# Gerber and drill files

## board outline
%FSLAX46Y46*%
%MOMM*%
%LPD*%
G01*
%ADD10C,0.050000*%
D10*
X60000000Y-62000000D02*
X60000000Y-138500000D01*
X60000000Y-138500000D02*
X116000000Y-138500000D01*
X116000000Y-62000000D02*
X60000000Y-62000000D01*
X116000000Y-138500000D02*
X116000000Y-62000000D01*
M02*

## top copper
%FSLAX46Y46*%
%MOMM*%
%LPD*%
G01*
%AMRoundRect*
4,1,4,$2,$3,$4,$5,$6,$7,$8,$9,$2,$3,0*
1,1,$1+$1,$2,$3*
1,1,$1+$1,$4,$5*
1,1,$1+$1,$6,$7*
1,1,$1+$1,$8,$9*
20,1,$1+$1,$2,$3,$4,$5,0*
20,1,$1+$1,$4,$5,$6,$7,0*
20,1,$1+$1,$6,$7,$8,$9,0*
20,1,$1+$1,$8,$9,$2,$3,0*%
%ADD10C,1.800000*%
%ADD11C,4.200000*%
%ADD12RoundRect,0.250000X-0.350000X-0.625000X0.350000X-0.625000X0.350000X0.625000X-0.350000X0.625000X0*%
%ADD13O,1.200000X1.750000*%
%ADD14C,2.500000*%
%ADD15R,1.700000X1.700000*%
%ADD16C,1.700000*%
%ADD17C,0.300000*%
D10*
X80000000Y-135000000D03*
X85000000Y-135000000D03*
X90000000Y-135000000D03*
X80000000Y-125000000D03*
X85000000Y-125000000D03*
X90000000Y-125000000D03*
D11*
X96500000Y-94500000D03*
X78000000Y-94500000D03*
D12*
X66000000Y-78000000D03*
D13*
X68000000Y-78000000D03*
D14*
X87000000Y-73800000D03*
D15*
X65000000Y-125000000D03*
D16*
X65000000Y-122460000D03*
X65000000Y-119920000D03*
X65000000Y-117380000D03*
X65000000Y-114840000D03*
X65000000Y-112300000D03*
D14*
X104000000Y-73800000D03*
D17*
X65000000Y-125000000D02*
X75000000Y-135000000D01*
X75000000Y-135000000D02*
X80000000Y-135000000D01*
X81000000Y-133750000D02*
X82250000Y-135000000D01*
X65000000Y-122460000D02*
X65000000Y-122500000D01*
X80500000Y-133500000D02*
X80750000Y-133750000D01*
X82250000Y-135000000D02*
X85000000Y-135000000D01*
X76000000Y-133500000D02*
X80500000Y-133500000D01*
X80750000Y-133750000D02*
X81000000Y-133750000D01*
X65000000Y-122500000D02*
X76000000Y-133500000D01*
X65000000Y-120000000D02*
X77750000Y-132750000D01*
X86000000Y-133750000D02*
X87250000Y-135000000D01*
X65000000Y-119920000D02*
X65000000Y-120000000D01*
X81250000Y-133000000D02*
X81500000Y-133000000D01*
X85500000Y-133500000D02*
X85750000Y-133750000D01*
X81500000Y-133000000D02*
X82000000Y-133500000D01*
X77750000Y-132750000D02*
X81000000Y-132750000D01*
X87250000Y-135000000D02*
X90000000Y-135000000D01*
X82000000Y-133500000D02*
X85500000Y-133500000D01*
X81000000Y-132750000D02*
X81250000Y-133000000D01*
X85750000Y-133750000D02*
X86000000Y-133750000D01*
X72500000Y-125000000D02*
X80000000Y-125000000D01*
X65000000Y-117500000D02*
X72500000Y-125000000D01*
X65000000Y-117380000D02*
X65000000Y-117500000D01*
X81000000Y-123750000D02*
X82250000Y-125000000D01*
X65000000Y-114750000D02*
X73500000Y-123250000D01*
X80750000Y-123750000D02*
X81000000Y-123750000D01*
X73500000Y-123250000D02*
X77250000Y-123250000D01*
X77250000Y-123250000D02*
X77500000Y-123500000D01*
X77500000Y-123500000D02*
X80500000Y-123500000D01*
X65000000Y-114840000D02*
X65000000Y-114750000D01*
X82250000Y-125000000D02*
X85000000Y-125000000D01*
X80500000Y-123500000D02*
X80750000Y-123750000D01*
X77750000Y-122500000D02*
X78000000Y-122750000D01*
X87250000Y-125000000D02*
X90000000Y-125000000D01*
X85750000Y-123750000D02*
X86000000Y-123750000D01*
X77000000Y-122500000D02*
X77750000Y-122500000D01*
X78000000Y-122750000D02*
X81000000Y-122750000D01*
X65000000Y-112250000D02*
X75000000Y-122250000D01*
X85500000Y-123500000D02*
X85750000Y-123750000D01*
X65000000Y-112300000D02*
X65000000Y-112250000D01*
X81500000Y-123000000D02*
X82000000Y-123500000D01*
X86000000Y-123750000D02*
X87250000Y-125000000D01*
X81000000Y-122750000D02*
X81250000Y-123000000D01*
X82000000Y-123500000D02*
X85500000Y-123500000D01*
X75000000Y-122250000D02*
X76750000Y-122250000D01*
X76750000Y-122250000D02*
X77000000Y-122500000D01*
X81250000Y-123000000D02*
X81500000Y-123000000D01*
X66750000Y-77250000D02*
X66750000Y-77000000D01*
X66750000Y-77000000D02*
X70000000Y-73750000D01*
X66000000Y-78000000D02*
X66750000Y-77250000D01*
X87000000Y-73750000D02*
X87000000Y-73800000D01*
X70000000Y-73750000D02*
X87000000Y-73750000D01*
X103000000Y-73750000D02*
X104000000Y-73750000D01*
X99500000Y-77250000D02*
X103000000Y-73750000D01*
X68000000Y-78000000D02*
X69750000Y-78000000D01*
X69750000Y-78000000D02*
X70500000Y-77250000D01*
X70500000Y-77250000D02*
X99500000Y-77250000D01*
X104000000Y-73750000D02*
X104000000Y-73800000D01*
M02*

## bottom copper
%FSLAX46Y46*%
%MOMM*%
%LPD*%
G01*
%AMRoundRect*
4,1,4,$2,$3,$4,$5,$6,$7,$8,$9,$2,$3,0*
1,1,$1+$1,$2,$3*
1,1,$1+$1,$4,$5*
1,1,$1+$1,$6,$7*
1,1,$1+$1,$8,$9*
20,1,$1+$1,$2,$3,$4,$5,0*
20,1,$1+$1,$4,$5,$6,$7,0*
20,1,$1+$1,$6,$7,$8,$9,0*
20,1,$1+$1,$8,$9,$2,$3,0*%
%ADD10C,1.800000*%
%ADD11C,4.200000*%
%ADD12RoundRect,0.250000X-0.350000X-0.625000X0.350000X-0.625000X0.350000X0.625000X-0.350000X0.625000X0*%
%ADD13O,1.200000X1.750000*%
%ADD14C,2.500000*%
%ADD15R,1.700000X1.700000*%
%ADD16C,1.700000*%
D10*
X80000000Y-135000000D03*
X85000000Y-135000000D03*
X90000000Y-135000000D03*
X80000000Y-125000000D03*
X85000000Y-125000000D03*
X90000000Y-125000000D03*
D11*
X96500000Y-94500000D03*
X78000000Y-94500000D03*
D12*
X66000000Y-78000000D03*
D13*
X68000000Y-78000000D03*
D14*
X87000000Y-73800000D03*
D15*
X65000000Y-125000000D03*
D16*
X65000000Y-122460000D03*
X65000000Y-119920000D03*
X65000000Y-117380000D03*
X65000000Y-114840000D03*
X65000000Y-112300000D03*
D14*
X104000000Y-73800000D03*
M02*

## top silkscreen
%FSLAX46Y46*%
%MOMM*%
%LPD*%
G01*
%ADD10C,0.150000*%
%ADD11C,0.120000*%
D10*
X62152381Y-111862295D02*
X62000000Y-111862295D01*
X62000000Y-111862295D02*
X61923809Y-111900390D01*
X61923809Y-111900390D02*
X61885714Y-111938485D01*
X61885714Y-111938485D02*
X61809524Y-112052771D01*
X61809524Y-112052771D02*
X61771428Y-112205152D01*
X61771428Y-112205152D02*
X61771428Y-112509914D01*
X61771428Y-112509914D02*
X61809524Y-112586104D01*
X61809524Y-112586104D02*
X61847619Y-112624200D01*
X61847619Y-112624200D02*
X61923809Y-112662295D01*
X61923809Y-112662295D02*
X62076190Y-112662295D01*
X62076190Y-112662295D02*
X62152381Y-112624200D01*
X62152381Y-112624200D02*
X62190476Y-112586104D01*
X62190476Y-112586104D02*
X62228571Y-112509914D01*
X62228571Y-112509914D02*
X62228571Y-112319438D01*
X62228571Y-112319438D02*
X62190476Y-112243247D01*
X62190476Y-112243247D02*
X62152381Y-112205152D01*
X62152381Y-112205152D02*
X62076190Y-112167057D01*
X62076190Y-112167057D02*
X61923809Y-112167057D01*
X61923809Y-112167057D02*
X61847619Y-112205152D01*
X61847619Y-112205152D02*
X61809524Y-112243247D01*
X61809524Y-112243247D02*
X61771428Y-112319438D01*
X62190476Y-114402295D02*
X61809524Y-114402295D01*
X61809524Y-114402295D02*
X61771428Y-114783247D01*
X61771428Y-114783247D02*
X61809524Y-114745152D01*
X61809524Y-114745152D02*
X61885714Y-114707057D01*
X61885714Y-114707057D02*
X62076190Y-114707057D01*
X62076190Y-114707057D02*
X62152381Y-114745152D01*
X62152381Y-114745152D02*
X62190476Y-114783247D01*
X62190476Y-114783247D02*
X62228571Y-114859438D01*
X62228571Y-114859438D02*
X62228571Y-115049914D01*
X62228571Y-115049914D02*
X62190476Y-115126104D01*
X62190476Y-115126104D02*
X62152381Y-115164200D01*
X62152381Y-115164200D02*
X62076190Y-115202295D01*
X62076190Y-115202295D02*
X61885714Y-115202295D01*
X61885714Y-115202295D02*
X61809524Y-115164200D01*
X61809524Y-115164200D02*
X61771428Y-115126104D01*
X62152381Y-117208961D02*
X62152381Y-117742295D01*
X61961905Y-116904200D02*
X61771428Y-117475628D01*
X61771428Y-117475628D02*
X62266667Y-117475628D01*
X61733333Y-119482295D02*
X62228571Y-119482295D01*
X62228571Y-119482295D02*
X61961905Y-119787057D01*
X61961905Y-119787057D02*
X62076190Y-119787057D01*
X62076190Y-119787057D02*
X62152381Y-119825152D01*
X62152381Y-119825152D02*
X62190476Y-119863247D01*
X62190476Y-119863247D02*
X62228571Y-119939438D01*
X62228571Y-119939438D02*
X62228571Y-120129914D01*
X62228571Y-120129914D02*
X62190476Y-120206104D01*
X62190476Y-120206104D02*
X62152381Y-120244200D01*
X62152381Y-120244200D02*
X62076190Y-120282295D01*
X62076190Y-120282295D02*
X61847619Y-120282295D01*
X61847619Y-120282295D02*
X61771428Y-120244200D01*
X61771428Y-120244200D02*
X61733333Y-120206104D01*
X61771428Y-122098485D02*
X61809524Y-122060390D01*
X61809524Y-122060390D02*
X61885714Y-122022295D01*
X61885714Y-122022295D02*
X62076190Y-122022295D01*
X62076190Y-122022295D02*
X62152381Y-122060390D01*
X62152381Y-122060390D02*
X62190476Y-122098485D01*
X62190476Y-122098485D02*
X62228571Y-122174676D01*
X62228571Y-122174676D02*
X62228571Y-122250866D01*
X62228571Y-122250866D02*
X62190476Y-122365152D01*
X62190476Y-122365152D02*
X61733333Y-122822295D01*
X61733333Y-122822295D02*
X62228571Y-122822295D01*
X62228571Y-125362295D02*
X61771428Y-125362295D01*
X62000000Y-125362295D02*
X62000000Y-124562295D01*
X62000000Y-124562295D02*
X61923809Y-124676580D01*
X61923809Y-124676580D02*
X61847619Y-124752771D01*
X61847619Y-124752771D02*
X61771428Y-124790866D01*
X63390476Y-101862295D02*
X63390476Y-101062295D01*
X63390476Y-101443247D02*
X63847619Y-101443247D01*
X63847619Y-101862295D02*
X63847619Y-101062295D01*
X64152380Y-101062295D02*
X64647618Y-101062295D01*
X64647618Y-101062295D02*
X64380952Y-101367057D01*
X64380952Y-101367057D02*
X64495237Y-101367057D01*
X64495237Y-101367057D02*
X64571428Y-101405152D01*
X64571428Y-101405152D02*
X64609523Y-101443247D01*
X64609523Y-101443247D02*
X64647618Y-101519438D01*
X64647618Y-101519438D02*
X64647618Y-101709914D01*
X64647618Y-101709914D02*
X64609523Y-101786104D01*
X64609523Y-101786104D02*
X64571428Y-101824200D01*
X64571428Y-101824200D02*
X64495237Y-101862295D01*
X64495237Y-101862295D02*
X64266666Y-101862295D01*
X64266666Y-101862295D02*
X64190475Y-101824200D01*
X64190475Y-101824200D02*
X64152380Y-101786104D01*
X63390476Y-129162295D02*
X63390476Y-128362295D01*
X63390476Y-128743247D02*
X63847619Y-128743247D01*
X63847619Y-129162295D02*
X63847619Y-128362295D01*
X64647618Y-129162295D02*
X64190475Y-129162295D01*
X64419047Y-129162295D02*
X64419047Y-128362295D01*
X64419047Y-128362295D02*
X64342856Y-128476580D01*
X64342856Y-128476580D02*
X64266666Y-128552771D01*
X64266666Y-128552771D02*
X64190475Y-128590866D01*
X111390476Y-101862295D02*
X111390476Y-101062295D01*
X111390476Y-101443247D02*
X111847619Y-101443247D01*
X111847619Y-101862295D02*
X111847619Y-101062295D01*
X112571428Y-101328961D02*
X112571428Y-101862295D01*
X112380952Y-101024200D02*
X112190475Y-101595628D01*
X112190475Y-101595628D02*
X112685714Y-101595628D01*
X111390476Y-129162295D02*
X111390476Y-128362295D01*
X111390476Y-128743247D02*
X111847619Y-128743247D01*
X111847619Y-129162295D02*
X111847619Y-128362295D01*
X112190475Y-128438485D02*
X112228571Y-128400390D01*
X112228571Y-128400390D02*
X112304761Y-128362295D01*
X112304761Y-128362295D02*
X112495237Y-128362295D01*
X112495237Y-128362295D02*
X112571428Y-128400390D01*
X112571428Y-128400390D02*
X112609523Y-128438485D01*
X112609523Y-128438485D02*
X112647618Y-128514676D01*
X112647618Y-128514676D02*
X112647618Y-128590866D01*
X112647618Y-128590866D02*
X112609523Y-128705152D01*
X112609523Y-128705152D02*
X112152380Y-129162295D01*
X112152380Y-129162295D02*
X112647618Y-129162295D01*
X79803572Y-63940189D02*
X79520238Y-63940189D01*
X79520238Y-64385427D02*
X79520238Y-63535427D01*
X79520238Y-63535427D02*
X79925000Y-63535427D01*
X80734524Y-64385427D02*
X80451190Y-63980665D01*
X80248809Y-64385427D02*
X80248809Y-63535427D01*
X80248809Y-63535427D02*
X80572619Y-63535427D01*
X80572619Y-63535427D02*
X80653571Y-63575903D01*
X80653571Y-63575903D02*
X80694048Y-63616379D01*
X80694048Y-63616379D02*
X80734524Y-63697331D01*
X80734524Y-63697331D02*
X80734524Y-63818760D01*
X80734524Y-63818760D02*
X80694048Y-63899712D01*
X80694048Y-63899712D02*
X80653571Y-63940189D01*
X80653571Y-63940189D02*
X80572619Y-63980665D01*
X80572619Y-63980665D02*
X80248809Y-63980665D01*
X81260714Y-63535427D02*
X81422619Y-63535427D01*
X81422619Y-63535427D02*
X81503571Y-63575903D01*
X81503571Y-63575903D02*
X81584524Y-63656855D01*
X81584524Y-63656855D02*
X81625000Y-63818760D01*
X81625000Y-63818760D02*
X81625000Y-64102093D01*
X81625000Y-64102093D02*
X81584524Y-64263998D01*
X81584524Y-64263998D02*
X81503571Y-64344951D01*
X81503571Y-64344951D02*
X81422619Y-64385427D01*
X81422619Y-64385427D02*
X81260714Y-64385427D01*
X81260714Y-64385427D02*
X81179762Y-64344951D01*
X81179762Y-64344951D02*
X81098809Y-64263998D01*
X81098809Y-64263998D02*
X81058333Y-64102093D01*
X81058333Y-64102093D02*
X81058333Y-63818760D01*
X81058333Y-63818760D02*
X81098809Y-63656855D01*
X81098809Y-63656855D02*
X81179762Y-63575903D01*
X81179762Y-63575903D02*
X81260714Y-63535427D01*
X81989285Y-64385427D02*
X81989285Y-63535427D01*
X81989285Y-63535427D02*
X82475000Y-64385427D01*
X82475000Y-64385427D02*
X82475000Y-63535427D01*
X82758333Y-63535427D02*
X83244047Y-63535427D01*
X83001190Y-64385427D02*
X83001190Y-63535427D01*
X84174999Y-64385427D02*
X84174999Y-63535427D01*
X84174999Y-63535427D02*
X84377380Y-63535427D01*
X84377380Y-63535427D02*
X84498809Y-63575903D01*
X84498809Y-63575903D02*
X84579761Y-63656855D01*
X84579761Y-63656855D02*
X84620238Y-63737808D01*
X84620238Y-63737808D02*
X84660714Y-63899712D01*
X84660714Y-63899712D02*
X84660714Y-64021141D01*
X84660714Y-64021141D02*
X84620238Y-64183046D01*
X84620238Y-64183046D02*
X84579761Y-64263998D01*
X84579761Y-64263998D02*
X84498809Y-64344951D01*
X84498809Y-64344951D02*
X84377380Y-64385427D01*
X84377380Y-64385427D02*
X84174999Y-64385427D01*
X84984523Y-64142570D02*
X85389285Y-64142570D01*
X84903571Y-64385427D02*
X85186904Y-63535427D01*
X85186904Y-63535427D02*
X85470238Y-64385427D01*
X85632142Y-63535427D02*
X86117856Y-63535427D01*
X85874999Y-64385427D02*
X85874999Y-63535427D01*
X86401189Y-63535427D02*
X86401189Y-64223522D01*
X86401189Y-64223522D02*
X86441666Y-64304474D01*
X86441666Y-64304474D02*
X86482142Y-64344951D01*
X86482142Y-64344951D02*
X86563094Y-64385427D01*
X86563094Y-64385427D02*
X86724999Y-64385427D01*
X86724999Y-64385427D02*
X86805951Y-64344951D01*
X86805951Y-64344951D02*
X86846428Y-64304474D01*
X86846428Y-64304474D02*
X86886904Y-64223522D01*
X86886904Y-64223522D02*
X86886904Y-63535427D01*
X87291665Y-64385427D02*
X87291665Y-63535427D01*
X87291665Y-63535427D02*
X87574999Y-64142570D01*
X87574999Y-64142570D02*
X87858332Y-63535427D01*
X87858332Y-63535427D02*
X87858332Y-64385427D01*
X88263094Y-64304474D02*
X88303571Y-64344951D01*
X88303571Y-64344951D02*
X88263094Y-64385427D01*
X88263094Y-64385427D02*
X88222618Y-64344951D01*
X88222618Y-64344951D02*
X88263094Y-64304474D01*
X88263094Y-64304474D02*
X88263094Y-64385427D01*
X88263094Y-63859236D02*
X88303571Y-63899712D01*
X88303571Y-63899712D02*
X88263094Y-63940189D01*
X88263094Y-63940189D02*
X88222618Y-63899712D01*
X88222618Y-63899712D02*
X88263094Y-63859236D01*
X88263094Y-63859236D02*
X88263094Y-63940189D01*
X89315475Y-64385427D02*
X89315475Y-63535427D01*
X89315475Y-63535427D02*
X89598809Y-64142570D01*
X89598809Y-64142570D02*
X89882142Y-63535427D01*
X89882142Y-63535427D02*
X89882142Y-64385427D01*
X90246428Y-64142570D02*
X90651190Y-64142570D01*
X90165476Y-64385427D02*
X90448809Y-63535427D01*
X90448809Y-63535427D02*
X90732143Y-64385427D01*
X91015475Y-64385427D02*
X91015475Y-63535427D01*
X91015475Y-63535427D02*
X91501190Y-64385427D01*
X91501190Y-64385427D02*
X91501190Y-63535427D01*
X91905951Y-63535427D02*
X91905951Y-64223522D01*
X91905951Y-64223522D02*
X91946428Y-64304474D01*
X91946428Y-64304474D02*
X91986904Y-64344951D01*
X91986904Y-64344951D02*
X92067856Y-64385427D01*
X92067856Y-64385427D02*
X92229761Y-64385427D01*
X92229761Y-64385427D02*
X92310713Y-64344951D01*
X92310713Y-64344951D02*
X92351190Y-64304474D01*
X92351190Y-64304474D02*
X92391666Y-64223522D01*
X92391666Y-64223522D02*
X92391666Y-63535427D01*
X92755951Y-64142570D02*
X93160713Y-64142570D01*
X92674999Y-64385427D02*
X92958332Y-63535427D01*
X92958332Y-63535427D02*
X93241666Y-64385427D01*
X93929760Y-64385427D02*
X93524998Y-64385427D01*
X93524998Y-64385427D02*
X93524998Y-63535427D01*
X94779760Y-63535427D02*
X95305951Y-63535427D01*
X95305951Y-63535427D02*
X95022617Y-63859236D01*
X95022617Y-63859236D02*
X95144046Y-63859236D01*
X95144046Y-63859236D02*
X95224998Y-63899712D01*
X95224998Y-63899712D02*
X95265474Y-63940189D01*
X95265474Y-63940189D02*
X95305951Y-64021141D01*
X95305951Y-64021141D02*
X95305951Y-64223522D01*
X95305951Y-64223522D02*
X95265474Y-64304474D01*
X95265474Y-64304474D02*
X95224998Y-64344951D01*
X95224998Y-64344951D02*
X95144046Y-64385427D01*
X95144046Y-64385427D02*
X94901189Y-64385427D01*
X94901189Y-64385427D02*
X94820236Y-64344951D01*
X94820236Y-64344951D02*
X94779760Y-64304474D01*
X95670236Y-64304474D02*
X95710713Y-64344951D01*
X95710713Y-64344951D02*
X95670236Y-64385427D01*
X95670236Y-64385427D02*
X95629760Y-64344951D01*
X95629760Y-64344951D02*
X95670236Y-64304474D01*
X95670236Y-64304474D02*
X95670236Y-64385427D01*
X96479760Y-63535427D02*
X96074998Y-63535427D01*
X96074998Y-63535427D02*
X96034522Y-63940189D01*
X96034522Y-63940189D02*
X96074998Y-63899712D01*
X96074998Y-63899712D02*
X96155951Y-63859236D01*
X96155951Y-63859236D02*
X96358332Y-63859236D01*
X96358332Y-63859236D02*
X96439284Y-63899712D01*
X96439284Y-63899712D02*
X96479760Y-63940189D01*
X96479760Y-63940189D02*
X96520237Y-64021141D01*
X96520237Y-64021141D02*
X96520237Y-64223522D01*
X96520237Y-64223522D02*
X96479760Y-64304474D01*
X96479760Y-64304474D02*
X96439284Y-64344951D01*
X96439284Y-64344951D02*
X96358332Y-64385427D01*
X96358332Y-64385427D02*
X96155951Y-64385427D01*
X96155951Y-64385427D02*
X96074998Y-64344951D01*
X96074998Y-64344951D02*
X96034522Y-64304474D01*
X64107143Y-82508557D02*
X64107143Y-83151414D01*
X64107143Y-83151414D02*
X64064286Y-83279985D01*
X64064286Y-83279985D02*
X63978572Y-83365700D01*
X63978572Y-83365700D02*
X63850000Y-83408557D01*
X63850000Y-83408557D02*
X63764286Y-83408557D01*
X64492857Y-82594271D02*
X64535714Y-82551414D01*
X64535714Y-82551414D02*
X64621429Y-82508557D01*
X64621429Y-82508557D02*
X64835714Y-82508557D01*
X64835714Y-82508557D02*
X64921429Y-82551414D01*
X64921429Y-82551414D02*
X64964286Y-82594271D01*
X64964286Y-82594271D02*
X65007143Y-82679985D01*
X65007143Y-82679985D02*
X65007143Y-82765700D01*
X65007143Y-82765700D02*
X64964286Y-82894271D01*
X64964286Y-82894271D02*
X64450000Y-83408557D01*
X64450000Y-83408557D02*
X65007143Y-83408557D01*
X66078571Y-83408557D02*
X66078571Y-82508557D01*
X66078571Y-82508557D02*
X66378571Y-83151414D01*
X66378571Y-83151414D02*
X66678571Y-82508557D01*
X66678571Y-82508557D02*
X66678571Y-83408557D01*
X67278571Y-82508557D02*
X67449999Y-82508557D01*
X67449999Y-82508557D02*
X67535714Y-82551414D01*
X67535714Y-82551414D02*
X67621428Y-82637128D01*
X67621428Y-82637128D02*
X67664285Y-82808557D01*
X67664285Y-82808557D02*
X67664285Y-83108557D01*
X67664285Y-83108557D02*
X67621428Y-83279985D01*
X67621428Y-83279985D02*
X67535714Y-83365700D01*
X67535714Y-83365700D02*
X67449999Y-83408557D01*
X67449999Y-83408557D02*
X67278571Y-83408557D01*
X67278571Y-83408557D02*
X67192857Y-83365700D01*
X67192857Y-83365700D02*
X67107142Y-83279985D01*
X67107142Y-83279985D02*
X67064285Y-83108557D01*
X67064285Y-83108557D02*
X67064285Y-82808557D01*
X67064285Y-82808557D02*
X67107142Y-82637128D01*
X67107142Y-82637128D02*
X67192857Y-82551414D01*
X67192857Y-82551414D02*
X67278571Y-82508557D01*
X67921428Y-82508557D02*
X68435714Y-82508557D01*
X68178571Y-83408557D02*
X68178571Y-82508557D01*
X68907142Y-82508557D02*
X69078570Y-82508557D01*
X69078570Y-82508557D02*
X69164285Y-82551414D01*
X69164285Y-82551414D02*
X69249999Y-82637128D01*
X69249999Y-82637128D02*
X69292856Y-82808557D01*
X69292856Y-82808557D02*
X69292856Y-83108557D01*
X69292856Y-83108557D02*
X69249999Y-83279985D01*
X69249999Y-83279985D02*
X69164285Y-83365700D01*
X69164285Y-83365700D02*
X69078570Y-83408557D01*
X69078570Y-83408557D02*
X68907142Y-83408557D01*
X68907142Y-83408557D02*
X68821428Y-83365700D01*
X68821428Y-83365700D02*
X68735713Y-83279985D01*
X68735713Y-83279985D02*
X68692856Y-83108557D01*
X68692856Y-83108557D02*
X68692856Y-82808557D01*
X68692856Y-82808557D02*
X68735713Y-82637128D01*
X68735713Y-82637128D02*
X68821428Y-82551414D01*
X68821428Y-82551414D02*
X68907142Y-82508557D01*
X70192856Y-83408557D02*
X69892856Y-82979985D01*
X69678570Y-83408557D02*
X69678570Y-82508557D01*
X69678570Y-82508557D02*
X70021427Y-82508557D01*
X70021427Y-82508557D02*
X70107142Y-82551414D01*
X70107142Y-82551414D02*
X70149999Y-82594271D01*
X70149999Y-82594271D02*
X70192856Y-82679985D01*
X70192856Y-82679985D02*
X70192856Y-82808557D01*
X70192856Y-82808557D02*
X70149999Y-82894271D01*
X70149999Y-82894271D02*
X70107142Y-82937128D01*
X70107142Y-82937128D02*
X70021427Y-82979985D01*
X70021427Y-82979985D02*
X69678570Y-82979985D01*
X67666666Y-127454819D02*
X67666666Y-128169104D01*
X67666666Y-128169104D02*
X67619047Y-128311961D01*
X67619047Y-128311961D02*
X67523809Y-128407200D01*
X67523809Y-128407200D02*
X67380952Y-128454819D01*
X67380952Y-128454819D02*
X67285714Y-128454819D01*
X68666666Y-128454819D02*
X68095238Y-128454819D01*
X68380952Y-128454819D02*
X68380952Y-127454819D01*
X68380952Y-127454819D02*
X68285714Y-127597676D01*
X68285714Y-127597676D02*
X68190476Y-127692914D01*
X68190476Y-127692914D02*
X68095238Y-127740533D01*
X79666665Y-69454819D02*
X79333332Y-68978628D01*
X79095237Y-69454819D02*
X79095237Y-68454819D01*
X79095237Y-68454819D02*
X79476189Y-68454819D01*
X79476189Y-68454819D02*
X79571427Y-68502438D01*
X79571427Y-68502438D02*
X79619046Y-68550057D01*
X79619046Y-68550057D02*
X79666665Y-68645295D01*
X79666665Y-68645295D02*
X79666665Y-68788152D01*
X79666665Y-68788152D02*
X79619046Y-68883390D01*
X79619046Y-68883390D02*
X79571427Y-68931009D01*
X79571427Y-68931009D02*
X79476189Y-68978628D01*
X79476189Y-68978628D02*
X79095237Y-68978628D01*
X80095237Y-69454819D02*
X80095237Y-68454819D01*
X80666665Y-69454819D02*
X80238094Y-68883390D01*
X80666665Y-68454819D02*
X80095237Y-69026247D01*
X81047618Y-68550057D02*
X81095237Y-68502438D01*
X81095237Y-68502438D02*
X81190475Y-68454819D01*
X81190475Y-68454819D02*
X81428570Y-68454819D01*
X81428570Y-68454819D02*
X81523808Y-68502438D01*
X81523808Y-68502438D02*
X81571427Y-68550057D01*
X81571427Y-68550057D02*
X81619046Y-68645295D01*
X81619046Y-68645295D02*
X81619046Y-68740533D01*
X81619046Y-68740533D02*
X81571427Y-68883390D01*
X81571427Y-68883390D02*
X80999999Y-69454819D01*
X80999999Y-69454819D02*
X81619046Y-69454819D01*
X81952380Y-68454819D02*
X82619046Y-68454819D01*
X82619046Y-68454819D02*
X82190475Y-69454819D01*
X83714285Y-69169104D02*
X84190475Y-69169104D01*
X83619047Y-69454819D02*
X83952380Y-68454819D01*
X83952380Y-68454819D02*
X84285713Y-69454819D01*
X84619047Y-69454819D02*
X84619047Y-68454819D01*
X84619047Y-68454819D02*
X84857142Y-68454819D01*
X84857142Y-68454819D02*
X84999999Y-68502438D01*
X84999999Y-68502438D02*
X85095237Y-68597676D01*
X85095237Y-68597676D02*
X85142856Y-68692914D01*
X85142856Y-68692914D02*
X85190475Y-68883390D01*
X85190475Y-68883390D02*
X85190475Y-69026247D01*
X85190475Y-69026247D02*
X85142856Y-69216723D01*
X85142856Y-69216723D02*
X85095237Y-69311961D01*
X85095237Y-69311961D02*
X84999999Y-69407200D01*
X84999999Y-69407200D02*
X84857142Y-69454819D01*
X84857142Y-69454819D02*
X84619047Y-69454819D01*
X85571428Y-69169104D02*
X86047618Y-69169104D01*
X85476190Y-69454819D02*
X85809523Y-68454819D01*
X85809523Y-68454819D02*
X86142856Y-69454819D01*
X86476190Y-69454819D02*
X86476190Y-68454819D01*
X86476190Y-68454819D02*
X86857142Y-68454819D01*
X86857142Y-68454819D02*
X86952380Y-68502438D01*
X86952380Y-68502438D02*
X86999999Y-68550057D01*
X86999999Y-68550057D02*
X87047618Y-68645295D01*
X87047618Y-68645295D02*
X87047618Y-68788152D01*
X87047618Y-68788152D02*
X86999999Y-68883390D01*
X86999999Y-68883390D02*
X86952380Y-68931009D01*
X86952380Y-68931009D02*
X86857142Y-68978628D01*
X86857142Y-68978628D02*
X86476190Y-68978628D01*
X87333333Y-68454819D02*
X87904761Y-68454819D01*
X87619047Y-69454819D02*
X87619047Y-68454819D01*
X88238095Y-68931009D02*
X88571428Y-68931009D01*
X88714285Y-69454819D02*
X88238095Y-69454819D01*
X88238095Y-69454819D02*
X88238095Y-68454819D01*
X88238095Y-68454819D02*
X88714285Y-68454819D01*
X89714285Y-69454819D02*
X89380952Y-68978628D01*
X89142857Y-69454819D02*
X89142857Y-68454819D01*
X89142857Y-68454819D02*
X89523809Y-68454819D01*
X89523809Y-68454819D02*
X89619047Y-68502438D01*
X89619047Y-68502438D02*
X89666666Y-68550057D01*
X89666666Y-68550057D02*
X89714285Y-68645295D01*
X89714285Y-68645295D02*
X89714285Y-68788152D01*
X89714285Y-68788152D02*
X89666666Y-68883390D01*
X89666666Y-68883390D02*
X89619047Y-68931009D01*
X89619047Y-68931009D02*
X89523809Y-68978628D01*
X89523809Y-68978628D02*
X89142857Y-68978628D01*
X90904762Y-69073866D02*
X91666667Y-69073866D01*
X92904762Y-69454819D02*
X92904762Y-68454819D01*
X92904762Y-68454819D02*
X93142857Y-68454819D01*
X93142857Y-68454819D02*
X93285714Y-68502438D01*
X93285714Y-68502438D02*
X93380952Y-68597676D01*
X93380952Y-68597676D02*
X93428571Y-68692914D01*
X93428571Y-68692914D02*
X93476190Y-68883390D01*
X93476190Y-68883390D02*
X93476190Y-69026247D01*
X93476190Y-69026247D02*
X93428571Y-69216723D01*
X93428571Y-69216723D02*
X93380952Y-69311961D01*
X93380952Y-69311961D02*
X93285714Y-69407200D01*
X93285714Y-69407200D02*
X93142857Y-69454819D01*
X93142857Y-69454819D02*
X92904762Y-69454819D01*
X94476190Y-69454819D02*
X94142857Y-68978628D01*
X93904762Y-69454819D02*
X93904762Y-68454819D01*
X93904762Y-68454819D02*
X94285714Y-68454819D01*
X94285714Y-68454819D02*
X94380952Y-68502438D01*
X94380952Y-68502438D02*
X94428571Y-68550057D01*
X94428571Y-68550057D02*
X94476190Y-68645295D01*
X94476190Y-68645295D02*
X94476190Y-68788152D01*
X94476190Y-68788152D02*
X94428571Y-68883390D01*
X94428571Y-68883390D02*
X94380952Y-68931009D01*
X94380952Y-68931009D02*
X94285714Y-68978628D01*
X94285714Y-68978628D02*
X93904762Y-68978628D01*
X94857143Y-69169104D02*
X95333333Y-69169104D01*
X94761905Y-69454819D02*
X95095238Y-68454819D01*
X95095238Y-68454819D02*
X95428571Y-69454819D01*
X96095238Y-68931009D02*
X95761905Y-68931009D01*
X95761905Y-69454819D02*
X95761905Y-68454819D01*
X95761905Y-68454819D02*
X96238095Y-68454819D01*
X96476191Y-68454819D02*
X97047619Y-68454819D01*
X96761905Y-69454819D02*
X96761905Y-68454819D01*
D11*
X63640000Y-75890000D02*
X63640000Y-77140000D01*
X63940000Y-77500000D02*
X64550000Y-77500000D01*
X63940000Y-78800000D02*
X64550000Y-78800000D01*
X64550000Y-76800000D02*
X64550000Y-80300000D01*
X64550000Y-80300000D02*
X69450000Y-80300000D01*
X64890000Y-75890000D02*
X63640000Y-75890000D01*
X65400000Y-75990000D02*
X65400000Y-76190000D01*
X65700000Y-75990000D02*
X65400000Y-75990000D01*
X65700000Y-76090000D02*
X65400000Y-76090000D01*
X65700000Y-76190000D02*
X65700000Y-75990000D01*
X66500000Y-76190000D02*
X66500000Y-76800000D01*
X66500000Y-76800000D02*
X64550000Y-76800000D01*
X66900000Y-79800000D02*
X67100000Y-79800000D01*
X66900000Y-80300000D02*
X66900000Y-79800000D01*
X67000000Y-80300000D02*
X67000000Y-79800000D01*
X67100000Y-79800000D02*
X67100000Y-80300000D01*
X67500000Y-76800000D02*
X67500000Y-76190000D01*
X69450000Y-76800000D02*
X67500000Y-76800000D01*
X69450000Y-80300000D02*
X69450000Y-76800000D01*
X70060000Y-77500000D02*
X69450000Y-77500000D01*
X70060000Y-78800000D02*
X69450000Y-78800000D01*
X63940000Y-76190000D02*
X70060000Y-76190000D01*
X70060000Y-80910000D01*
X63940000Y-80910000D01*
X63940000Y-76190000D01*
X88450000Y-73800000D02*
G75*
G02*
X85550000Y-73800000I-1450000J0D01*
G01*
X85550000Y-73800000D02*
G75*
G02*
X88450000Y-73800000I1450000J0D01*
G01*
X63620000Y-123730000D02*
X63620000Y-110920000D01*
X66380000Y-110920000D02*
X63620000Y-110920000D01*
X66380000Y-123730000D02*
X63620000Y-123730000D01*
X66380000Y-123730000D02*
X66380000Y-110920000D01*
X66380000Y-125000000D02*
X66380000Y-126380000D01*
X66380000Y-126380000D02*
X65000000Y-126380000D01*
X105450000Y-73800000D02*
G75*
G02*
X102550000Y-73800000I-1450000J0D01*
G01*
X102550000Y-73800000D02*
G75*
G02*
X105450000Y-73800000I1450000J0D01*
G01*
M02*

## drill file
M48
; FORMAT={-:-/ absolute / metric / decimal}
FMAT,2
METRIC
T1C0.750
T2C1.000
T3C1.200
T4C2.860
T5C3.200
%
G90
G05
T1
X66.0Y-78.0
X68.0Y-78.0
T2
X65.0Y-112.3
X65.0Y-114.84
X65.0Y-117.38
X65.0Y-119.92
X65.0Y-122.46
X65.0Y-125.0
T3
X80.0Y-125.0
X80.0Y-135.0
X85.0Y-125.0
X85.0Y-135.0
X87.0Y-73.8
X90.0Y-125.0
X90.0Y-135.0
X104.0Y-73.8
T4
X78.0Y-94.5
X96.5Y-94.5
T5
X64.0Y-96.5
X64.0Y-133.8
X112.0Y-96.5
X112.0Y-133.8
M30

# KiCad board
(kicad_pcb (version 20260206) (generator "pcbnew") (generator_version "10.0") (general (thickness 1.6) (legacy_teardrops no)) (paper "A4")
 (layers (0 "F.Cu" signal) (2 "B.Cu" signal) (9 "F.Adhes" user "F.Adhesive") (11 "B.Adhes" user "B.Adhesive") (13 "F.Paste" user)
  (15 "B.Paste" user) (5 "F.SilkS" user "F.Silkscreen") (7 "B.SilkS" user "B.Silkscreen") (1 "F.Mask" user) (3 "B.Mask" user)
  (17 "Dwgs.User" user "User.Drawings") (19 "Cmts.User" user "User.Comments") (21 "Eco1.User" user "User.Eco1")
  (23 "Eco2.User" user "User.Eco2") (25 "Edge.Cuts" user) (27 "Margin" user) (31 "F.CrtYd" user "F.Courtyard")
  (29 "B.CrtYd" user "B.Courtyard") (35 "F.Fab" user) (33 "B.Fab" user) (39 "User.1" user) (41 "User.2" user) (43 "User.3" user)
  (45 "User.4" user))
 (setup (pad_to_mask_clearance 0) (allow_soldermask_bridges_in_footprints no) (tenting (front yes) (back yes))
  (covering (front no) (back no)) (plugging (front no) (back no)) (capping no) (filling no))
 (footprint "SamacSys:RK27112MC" (layer "F.Cu") (at 85 94.5 -90)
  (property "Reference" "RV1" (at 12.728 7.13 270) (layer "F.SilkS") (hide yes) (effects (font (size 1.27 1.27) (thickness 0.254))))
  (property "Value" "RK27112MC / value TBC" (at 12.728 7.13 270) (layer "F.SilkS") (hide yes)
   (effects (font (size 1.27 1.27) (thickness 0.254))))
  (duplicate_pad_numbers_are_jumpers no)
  (pad "1" thru_hole circle (at 40.5 5 270) (size 1.8 1.8) (drill 1.2) (layers "*.Cu" "*.Mask") (remove_unused_layers no) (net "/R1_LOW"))
  (pad "2" thru_hole circle (at 40.5 0 270) (size 1.8 1.8) (drill 1.2) (layers "*.Cu" "*.Mask") (remove_unused_layers no) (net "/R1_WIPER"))
  (pad "3" thru_hole circle (at 40.5 -5 270) (size 1.8 1.8) (drill 1.2) (layers "*.Cu" "*.Mask") (remove_unused_layers no) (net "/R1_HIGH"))
  (pad "4" thru_hole circle (at 30.5 5 270) (size 1.8 1.8) (drill 1.2) (layers "*.Cu" "*.Mask") (remove_unused_layers no) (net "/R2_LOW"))
  (pad "5" thru_hole circle (at 30.5 0 270) (size 1.8 1.8) (drill 1.2) (layers "*.Cu" "*.Mask") (remove_unused_layers no) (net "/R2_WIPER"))
  (pad "6" thru_hole circle (at 30.5 -5 270) (size 1.8 1.8) (drill 1.2) (layers "*.Cu" "*.Mask") (remove_unused_layers no) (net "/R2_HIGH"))
  (pad "7" thru_hole circle (at 0 -11.5 270) (size 4.2 4.2) (drill 2.86) (layers "*.Cu" "*.Mask") (remove_unused_layers no)
   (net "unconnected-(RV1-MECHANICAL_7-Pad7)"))
  (pad "8" thru_hole circle (at 0 7 270) (size 4.2 4.2) (drill 2.86) (layers "*.Cu" "*.Mask") (remove_unused_layers no)
   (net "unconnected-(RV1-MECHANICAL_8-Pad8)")))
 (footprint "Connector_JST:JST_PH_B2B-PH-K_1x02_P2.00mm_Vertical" (layer "F.Cu") (at 66 78)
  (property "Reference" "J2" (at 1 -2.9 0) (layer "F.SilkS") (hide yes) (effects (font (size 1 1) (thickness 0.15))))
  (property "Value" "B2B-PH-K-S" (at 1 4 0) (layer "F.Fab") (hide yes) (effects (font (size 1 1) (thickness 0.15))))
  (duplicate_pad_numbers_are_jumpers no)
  (fp_line (start -2.36 -2.11) (end -2.36 -0.86) (stroke (width 0.12) (type solid)) (layer "F.SilkS"))
  (fp_line (start -2.06 -0.5) (end -1.45 -0.5) (stroke (width 0.12) (type solid)) (layer "F.SilkS"))
  (fp_line (start -2.06 0.8) (end -1.45 0.8) (stroke (width 0.12) (type solid)) (layer "F.SilkS"))
  (fp_line (start -1.45 -1.2) (end -1.45 2.3) (stroke (width 0.12) (type solid)) (layer "F.SilkS"))
  (fp_line (start -1.45 2.3) (end 3.45 2.3) (stroke (width 0.12) (type solid)) (layer "F.SilkS"))
  (fp_line (start -1.11 -2.11) (end -2.36 -2.11) (stroke (width 0.12) (type solid)) (layer "F.SilkS"))
  (fp_line (start -0.6 -2.01) (end -0.6 -1.81) (stroke (width 0.12) (type solid)) (layer "F.SilkS"))
  (fp_line (start -0.3 -2.01) (end -0.6 -2.01) (stroke (width 0.12) (type solid)) (layer "F.SilkS"))
  (fp_line (start -0.3 -1.91) (end -0.6 -1.91) (stroke (width 0.12) (type solid)) (layer "F.SilkS"))
  (fp_line (start -0.3 -1.81) (end -0.3 -2.01) (stroke (width 0.12) (type solid)) (layer "F.SilkS"))
  (fp_line (start 0.5 -1.81) (end 0.5 -1.2) (stroke (width 0.12) (type solid)) (layer "F.SilkS"))
  (fp_line (start 0.5 -1.2) (end -1.45 -1.2) (stroke (width 0.12) (type solid)) (layer "F.SilkS"))
  (fp_line (start 0.9 1.8) (end 1.1 1.8) (stroke (width 0.12) (type solid)) (layer "F.SilkS"))
  (fp_line (start 0.9 2.3) (end 0.9 1.8) (stroke (width 0.12) (type solid)) (layer "F.SilkS"))
  (fp_line (start 1 2.3) (end 1 1.8) (stroke (width 0.12) (type solid)) (layer "F.SilkS"))
  (fp_line (start 1.1 1.8) (end 1.1 2.3) (stroke (width 0.12) (type solid)) (layer "F.SilkS"))
  (fp_line (start 1.5 -1.2) (end 1.5 -1.81) (stroke (width 0.12) (type solid)) (layer "F.SilkS"))
  (fp_line (start 3.45 -1.2) (end 1.5 -1.2) (stroke (width 0.12) (type solid)) (layer "F.SilkS"))
  (fp_line (start 3.45 2.3) (end 3.45 -1.2) (stroke (width 0.12) (type solid)) (layer "F.SilkS"))
  (fp_line (start 4.06 -0.5) (end 3.45 -0.5) (stroke (width 0.12) (type solid)) (layer "F.SilkS"))
  (fp_line (start 4.06 0.8) (end 3.45 0.8) (stroke (width 0.12) (type solid)) (layer "F.SilkS"))
  (fp_rect (start -2.06 -1.81) (end 4.06 2.91) (stroke (width 0.12) (type solid)) (fill no) (layer "F.SilkS"))
  (pad "1" thru_hole roundrect (at 0 0) (size 1.2 1.75) (drill 0.75) (layers "*.Cu" "*.Mask") (remove_unused_layers no)
   (roundrect_rratio 0.208333) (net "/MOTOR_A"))
  (pad "2" thru_hole oval (at 2 0) (size 1.2 1.75) (drill 0.75) (layers "*.Cu" "*.Mask") (remove_unused_layers no) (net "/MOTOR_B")))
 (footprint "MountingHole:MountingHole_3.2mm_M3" (layer "F.Cu") (at 112 133.8)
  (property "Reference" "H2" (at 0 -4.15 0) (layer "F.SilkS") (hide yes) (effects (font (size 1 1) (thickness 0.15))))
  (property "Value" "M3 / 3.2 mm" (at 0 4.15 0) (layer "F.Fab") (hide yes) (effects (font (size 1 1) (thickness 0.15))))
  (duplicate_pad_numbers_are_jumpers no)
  (pad "" np_thru_hole circle (at 0 0) (size 3.2 3.2) (drill 3.2) (layers "*.Cu" "*.Mask")))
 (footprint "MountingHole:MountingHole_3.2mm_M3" (layer "F.Cu") (at 64 96.5)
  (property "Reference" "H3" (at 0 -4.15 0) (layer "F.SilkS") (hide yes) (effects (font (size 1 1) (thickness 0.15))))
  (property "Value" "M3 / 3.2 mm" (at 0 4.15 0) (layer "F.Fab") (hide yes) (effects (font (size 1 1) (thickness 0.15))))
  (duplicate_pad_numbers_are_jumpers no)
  (pad "" np_thru_hole circle (at 0 0) (size 3.2 3.2) (drill 3.2) (layers "*.Cu" "*.Mask")))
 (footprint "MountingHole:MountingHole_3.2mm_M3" (layer "F.Cu") (at 64 133.8)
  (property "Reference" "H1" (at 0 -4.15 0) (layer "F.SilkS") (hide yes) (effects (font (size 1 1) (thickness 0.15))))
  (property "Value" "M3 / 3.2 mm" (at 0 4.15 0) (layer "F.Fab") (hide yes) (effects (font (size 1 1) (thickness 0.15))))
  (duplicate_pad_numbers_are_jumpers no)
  (pad "" np_thru_hole circle (at 0 0) (size 3.2 3.2) (drill 3.2) (layers "*.Cu" "*.Mask")))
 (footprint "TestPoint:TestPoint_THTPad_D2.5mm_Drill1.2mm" (layer "F.Cu") (at 87 73.8)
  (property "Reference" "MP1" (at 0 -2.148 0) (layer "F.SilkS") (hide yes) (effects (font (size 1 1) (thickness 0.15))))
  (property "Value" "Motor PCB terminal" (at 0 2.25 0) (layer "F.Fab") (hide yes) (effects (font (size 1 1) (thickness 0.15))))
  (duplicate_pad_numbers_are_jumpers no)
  (fp_circle (center 0 0) (end 0 1.45) (stroke (width 0.12) (type solid)) (fill no) (layer "F.SilkS"))
  (pad "1" thru_hole circle (at 0 0) (size 2.5 2.5) (drill 1.2) (layers "*.Cu" "*.Mask") (remove_unused_layers no) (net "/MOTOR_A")))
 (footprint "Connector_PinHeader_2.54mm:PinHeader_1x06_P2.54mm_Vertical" (layer "F.Cu") (at 65 125 180)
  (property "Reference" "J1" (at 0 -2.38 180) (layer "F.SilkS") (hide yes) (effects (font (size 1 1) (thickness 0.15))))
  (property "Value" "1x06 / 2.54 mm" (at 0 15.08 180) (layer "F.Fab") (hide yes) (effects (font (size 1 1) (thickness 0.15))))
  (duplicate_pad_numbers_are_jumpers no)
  (fp_line (start 1.38 1.27) (end 1.38 14.08) (stroke (width 0.12) (type solid)) (layer "F.SilkS"))
  (fp_line (start -1.38 14.08) (end 1.38 14.08) (stroke (width 0.12) (type solid)) (layer "F.SilkS"))
  (fp_line (start -1.38 1.27) (end 1.38 1.27) (stroke (width 0.12) (type solid)) (layer "F.SilkS"))
  (fp_line (start -1.38 1.27) (end -1.38 14.08) (stroke (width 0.12) (type solid)) (layer "F.SilkS"))
  (fp_line (start -1.38 0) (end -1.38 -1.38) (stroke (width 0.12) (type solid)) (layer "F.SilkS"))
  (fp_line (start -1.38 -1.38) (end 0 -1.38) (stroke (width 0.12) (type solid)) (layer "F.SilkS"))
  (pad "1" thru_hole rect (at 0 0 180) (size 1.7 1.7) (drill 1) (layers "*.Cu" "*.Mask") (remove_unused_layers no) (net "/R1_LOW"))
  (pad "2" thru_hole circle (at 0 2.54 180) (size 1.7 1.7) (drill 1) (layers "*.Cu" "*.Mask") (remove_unused_layers no) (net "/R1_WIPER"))
  (pad "3" thru_hole circle (at 0 5.08 180) (size 1.7 1.7) (drill 1) (layers "*.Cu" "*.Mask") (remove_unused_layers no) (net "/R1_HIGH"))
  (pad "4" thru_hole circle (at 0 7.62 180) (size 1.7 1.7) (drill 1) (layers "*.Cu" "*.Mask") (remove_unused_layers no) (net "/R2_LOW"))
  (pad "5" thru_hole circle (at 0 10.16 180) (size 1.7 1.7) (drill 1) (layers "*.Cu" "*.Mask") (remove_unused_layers no) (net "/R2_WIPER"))
  (pad "6" thru_hole circle (at 0 12.7 180) (size 1.7 1.7) (drill 1) (layers "*.Cu" "*.Mask") (remove_unused_layers no) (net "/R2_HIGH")))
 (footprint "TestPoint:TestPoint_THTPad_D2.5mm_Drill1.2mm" (layer "F.Cu") (at 104 73.8)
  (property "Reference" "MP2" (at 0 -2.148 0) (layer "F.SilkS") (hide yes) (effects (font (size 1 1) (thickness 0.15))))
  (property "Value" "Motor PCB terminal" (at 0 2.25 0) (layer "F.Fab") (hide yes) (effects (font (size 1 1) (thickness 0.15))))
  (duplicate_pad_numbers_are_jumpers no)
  (fp_circle (center 0 0) (end 0 1.45) (stroke (width 0.12) (type solid)) (fill no) (layer "F.SilkS"))
  (pad "1" thru_hole circle (at 0 0) (size 2.5 2.5) (drill 1.2) (layers "*.Cu" "*.Mask") (remove_unused_layers no) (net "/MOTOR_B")))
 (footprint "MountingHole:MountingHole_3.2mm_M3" (layer "F.Cu") (at 112 96.5)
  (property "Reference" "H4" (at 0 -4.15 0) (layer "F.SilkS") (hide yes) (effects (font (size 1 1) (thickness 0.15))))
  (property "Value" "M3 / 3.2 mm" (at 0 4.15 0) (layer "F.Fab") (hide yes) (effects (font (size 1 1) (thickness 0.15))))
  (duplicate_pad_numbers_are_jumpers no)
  (pad "" np_thru_hole circle (at 0 0) (size 3.2 3.2) (drill 3.2) (layers "*.Cu" "*.Mask")))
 (gr_line (start 60 62) (end 60 138.5) (stroke (width 0.05) (type default)) (layer "Edge.Cuts"))
 (gr_line (start 60 138.5) (end 116 138.5) (stroke (width 0.05) (type default)) (layer "Edge.Cuts"))
 (gr_line (start 116 62) (end 60 62) (stroke (width 0.05) (type default)) (layer "Edge.Cuts"))
 (gr_line (start 116 138.5) (end 116 62) (stroke (width 0.05) (type default)) (layer "Edge.Cuts"))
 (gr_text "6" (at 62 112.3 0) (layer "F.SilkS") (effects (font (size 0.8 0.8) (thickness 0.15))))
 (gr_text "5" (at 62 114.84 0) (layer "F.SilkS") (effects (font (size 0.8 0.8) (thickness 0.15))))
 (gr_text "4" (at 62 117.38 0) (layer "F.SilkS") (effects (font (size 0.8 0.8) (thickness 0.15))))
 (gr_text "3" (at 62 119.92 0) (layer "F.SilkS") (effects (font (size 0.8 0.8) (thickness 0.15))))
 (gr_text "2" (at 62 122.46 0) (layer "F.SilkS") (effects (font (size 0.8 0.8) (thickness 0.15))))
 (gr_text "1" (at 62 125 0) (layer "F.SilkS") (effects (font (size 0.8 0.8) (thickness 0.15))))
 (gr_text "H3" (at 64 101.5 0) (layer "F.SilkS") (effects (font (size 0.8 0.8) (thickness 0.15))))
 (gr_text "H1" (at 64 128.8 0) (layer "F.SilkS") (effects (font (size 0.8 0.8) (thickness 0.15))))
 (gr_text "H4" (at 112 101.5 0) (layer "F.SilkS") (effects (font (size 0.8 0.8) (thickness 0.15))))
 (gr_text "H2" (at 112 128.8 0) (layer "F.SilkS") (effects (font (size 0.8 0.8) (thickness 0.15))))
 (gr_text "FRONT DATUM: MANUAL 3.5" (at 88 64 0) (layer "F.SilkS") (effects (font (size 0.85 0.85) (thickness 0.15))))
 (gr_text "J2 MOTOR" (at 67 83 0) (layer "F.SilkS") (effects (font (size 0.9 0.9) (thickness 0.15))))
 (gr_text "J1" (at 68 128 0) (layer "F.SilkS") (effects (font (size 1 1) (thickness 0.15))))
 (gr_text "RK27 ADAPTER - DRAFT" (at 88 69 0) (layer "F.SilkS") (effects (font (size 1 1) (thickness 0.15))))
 (segment (start 65 125) (end 75 135) (width 0.3) (layer "F.Cu") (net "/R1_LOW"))
 (segment (start 75 135) (end 80 135) (width 0.3) (layer "F.Cu") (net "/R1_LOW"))
 (segment (start 81 133.75) (end 82.25 135) (width 0.3) (layer "F.Cu") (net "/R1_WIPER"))
 (segment (start 65 122.46) (end 65 122.5) (width 0.3) (layer "F.Cu") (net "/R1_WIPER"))
 (segment (start 80.5 133.5) (end 80.75 133.75) (width 0.3) (layer "F.Cu") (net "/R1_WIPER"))
 (segment (start 82.25 135) (end 85 135) (width 0.3) (layer "F.Cu") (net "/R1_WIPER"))
 (segment (start 76 133.5) (end 80.5 133.5) (width 0.3) (layer "F.Cu") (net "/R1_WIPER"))
 (segment (start 80.75 133.75) (end 81 133.75) (width 0.3) (layer "F.Cu") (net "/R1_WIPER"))
 (segment (start 65 122.5) (end 76 133.5) (width 0.3) (layer "F.Cu") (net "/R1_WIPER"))
 (segment (start 65 120) (end 77.75 132.75) (width 0.3) (layer "F.Cu") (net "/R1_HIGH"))
 (segment (start 86 133.75) (end 87.25 135) (width 0.3) (layer "F.Cu") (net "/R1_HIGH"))
 (segment (start 65 119.92) (end 65 120) (width 0.3) (layer "F.Cu") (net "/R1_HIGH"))
 (segment (start 81.25 133) (end 81.5 133) (width 0.3) (layer "F.Cu") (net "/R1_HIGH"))
 (segment (start 85.5 133.5) (end 85.75 133.75) (width 0.3) (layer "F.Cu") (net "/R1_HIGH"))
 (segment (start 81.5 133) (end 82 133.5) (width 0.3) (layer "F.Cu") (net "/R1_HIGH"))
 (segment (start 77.75 132.75) (end 81 132.75) (width 0.3) (layer "F.Cu") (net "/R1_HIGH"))
 (segment (start 87.25 135) (end 90 135) (width 0.3) (layer "F.Cu") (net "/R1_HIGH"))
 (segment (start 82 133.5) (end 85.5 133.5) (width 0.3) (layer "F.Cu") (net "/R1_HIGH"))
 (segment (start 81 132.75) (end 81.25 133) (width 0.3) (layer "F.Cu") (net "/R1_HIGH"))
 (segment (start 85.75 133.75) (end 86 133.75) (width 0.3) (layer "F.Cu") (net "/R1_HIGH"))
 (segment (start 72.5 125) (end 80 125) (width 0.3) (layer "F.Cu") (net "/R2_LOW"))
 (segment (start 65 117.5) (end 72.5 125) (width 0.3) (layer "F.Cu") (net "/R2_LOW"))
 (segment (start 65 117.38) (end 65 117.5) (width 0.3) (layer "F.Cu") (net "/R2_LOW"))
 (segment (start 81 123.75) (end 82.25 125) (width 0.3) (layer "F.Cu") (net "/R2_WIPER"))
 (segment (start 65 114.75) (end 73.5 123.25) (width 0.3) (layer "F.Cu") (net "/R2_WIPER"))
 (segment (start 80.75 123.75) (end 81 123.75) (width 0.3) (layer "F.Cu") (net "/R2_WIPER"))
 (segment (start 73.5 123.25) (end 77.25 123.25) (width 0.3) (layer "F.Cu") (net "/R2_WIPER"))
 (segment (start 77.25 123.25) (end 77.5 123.5) (width 0.3) (layer "F.Cu") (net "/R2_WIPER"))
 (segment (start 77.5 123.5) (end 80.5 123.5) (width 0.3) (layer "F.Cu") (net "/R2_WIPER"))
 (segment (start 65 114.84) (end 65 114.75) (width 0.3) (layer "F.Cu") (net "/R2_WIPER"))
 (segment (start 82.25 125) (end 85 125) (width 0.3) (layer "F.Cu") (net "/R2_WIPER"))
 (segment (start 80.5 123.5) (end 80.75 123.75) (width 0.3) (layer "F.Cu") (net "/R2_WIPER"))
 (segment (start 77.75 122.5) (end 78 122.75) (width 0.3) (layer "F.Cu") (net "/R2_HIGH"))
 (segment (start 87.25 125) (end 90 125) (width 0.3) (layer "F.Cu") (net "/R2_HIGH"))
 (segment (start 85.75 123.75) (end 86 123.75) (width 0.3) (layer "F.Cu") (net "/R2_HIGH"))
 (segment (start 77 122.5) (end 77.75 122.5) (width 0.3) (layer "F.Cu") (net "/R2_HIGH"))
 (segment (start 78 122.75) (end 81 122.75) (width 0.3) (layer "F.Cu") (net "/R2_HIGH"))
 (segment (start 65 112.25) (end 75 122.25) (width 0.3) (layer "F.Cu") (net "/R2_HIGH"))
 (segment (start 85.5 123.5) (end 85.75 123.75) (width 0.3) (layer "F.Cu") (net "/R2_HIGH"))
 (segment (start 65 112.3) (end 65 112.25) (width 0.3) (layer "F.Cu") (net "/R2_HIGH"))
 (segment (start 81.5 123) (end 82 123.5) (width 0.3) (layer "F.Cu") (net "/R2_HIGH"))
 (segment (start 86 123.75) (end 87.25 125) (width 0.3) (layer "F.Cu") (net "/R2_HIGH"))
 (segment (start 81 122.75) (end 81.25 123) (width 0.3) (layer "F.Cu") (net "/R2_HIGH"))
 (segment (start 82 123.5) (end 85.5 123.5) (width 0.3) (layer "F.Cu") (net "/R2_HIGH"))
 (segment (start 75 122.25) (end 76.75 122.25) (width 0.3) (layer "F.Cu") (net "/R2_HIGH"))
 (segment (start 76.75 122.25) (end 77 122.5) (width 0.3) (layer "F.Cu") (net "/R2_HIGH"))
 (segment (start 81.25 123) (end 81.5 123) (width 0.3) (layer "F.Cu") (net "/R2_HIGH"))
 (segment (start 66.75 77.25) (end 66.75 77) (width 0.3) (layer "F.Cu") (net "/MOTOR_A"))
 (segment (start 66.75 77) (end 70 73.75) (width 0.3) (layer "F.Cu") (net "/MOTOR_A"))
 (segment (start 66 78) (end 66.75 77.25) (width 0.3) (layer "F.Cu") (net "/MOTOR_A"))
 (segment (start 87 73.75) (end 87 73.8) (width 0.3) (layer "F.Cu") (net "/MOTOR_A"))
 (segment (start 70 73.75) (end 87 73.75) (width 0.3) (layer "F.Cu") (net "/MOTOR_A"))
 (segment (start 103 73.75) (end 104 73.75) (width 0.3) (layer "F.Cu") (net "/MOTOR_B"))
 (segment (start 99.5 77.25) (end 103 73.75) (width 0.3) (layer "F.Cu") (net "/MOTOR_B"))
 (segment (start 68 78) (end 69.75 78) (width 0.3) (layer "F.Cu") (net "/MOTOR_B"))
 (segment (start 69.75 78) (end 70.5 77.25) (width 0.3) (layer "F.Cu") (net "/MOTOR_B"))
 (segment (start 70.5 77.25) (end 99.5 77.25) (width 0.3) (layer "F.Cu") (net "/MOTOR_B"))
 (segment (start 104 73.75) (end 104 73.8) (width 0.3) (layer "F.Cu") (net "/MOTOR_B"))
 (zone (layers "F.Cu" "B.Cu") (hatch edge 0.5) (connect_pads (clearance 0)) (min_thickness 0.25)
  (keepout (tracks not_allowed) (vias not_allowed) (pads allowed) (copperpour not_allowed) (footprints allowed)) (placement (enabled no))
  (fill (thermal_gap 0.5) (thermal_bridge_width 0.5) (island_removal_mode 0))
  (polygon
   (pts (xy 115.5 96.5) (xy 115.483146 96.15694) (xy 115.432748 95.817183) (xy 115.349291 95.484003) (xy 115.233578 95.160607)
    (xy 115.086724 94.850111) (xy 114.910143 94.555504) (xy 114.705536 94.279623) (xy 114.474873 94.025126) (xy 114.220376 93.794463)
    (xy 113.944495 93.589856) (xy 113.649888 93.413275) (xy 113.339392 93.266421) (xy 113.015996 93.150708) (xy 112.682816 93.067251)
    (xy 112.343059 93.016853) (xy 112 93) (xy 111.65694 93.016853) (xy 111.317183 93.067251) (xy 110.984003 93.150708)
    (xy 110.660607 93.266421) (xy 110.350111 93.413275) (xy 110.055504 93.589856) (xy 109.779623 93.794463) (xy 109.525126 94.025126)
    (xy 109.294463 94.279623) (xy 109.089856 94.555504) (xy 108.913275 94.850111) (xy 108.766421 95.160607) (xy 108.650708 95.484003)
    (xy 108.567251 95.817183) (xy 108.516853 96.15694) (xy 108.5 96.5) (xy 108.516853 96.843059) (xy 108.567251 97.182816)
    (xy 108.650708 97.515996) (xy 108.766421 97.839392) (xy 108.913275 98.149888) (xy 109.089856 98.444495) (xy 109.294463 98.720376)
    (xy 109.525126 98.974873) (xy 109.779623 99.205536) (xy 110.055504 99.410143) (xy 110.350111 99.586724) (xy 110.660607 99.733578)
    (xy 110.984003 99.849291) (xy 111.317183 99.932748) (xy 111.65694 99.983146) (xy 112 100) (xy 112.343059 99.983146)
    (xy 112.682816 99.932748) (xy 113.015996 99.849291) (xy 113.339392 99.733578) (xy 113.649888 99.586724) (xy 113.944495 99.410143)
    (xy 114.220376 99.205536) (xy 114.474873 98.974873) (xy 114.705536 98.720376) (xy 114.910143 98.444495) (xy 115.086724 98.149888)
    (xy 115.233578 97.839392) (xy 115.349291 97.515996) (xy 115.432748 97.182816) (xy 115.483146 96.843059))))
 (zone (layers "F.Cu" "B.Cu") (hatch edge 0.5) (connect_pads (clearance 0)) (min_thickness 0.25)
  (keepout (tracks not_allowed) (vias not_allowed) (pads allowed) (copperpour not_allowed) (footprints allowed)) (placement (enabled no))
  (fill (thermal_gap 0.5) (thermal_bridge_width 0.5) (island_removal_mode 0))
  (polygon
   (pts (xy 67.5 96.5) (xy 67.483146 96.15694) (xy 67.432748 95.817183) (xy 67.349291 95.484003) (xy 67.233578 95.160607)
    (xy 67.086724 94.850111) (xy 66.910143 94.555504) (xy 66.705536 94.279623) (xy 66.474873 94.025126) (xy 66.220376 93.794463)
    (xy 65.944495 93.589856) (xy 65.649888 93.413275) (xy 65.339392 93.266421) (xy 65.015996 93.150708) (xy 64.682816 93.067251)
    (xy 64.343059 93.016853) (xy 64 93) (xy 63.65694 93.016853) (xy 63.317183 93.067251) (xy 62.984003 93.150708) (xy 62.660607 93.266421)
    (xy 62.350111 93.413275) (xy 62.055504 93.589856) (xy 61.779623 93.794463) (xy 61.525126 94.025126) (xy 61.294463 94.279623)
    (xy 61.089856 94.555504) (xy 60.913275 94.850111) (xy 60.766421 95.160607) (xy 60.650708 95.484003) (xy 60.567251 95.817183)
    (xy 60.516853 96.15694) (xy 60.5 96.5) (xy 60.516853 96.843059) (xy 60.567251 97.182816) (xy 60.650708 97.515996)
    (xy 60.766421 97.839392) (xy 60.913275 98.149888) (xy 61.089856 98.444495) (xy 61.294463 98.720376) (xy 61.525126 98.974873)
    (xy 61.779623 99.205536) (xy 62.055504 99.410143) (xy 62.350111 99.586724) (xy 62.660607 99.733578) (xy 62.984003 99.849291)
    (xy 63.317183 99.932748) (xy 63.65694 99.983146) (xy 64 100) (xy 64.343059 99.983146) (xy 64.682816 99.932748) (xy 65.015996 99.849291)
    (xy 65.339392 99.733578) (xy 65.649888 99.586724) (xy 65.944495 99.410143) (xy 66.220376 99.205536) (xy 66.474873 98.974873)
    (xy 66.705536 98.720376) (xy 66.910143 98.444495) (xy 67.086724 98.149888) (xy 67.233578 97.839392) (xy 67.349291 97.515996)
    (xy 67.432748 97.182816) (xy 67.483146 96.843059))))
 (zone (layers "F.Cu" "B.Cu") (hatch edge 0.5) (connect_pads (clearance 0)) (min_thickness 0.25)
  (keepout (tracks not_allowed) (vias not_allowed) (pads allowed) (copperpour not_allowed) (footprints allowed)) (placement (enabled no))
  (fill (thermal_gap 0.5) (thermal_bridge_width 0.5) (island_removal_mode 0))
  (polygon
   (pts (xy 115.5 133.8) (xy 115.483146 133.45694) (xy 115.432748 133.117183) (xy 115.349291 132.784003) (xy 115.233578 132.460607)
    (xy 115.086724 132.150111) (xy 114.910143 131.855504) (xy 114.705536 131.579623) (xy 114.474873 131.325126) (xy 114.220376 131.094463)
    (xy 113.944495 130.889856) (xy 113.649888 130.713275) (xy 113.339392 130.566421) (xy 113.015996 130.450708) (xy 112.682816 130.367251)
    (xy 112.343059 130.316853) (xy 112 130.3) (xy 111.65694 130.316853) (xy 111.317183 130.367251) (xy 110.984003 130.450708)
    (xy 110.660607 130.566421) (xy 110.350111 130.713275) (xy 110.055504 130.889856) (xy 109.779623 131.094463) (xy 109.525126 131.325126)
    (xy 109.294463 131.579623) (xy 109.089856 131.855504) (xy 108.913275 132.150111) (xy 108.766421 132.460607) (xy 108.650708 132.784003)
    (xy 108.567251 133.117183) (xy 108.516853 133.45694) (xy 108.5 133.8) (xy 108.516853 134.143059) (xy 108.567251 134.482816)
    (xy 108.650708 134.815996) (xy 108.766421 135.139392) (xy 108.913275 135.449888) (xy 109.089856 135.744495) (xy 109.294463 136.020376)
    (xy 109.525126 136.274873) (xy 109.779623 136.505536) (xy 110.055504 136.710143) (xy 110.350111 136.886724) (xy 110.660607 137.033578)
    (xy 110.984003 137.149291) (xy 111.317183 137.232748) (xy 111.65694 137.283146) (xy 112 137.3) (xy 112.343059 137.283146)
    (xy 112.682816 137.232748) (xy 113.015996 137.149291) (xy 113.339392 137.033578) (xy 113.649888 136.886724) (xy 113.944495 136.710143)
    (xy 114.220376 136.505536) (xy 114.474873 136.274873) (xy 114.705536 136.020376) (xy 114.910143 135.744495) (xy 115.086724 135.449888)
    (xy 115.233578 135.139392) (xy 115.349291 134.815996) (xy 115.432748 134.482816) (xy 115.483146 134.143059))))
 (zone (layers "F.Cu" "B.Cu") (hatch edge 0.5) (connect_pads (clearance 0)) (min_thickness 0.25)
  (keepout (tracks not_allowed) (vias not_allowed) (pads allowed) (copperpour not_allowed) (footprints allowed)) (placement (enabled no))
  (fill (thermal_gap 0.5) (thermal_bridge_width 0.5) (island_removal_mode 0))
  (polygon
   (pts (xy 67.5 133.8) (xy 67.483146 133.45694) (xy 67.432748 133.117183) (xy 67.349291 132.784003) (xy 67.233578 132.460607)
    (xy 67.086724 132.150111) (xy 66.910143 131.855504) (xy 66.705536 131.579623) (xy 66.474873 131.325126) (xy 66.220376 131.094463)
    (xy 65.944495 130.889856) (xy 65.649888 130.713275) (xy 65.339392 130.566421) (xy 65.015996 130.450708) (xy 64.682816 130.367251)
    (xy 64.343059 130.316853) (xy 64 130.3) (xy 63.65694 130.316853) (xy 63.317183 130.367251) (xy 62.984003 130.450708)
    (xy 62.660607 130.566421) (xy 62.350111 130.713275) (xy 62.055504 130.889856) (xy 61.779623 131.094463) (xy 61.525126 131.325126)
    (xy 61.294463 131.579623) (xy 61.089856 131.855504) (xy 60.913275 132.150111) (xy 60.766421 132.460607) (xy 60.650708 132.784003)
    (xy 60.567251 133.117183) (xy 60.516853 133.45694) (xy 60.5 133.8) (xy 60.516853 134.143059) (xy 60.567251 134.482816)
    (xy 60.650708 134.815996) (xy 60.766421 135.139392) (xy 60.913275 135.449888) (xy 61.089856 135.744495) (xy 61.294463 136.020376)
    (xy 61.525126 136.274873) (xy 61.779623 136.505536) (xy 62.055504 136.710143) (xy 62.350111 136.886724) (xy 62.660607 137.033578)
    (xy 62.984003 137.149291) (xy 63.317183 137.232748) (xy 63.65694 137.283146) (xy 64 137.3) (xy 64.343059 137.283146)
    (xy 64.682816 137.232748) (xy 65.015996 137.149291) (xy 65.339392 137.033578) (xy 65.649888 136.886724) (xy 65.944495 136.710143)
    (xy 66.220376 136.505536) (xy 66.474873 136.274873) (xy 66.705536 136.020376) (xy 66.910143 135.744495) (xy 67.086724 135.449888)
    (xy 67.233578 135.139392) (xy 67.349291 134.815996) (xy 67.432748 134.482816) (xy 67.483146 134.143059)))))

